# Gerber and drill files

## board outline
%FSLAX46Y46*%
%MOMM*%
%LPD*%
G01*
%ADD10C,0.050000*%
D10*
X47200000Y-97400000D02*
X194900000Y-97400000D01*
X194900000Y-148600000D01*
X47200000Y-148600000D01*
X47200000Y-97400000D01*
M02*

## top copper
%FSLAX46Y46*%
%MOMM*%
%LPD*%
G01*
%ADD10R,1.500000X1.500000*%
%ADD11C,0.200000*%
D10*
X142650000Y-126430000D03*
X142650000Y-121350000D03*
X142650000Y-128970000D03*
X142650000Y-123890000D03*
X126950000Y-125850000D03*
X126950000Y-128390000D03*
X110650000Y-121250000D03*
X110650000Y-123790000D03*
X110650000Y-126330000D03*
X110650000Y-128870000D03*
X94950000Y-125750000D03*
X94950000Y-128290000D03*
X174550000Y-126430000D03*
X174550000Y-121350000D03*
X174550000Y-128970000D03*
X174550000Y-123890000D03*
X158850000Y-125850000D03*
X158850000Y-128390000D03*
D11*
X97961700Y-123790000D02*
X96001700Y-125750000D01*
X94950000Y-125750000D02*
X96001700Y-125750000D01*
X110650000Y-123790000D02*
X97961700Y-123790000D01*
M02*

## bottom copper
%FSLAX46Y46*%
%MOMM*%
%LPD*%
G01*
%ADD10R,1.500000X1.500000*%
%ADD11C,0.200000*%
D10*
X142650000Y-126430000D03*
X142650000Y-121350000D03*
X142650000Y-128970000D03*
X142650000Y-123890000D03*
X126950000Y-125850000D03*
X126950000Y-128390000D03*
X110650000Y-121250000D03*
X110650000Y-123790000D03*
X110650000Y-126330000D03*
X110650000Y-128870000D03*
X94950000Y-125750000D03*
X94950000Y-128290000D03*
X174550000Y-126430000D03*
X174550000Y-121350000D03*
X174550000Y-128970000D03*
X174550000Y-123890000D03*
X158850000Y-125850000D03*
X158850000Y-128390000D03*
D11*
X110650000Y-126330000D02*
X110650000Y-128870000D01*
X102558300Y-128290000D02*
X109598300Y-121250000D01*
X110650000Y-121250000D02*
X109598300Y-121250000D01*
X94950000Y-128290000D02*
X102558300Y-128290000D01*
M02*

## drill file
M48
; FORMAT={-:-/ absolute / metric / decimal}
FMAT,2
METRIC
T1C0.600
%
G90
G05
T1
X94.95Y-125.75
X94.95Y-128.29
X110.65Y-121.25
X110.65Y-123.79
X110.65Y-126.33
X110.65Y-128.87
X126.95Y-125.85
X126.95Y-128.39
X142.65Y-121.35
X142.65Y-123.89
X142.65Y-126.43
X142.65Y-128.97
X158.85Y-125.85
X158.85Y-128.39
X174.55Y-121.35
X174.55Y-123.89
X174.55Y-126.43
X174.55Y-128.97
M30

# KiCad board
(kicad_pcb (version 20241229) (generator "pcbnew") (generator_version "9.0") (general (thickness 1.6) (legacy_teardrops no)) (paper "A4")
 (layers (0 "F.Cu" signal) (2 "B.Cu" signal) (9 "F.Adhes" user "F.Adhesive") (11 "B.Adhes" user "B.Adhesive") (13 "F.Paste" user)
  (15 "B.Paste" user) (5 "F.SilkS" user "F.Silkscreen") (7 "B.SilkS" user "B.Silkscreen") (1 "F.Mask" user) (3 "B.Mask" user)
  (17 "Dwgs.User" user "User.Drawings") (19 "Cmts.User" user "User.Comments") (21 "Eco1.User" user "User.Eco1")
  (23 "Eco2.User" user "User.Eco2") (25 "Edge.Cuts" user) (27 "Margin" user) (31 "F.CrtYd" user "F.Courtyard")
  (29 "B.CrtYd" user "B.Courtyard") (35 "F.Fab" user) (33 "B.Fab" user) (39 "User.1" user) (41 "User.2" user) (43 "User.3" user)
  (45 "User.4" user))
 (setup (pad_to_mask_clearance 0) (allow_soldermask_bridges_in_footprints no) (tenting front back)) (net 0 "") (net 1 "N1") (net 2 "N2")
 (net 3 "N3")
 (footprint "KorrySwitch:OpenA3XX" (layer "F.Cu") (at 124.75 116.85)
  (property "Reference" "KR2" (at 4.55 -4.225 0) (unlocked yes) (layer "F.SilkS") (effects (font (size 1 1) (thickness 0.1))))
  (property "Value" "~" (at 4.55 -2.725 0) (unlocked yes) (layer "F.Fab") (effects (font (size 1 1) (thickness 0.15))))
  (pad "5V_BL" thru_hole rect (at 17.9 9.58) (size 1.5 1.5) (drill 0.6) (layers "*.Cu" "*.Mask") (remove_unused_layers no))
  (pad "5V_TL" thru_hole rect (at 17.9 4.5) (size 1.5 1.5) (drill 0.6) (layers "*.Cu" "*.Mask") (remove_unused_layers no))
  (pad "GND_BL" thru_hole rect (at 17.9 12.12) (size 1.5 1.5) (drill 0.6) (layers "*.Cu" "*.Mask") (remove_unused_layers no))
  (pad "GND_TL" thru_hole rect (at 17.9 7.04) (size 1.5 1.5) (drill 0.6) (layers "*.Cu" "*.Mask") (remove_unused_layers no))
  (pad "SW_IN" thru_hole rect (at 2.2 9) (size 1.5 1.5) (drill 0.6) (layers "*.Cu" "*.Mask") (remove_unused_layers no))
  (pad "SW_OUT" thru_hole rect (at 2.2 11.54) (size 1.5 1.5) (drill 0.6) (layers "*.Cu" "*.Mask") (remove_unused_layers no)))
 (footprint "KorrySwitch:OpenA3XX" (layer "F.Cu") (at 92.75 116.75)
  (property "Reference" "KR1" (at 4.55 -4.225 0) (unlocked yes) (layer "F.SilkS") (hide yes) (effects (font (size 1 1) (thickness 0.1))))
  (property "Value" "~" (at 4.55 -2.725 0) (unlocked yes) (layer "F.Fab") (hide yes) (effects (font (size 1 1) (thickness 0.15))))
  (pad "1" thru_hole rect (at 17.9 4.5) (size 1.5 1.5) (drill 0.6) (layers "*.Cu" "*.Mask") (remove_unused_layers no) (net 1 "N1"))
  (pad "2" thru_hole rect (at 17.9 7.04) (size 1.5 1.5) (drill 0.6) (layers "*.Cu" "*.Mask") (remove_unused_layers no) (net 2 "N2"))
  (pad "3" thru_hole rect (at 17.9 9.58) (size 1.5 1.5) (drill 0.6) (layers "*.Cu" "*.Mask") (remove_unused_layers no) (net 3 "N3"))
  (pad "4" thru_hole rect (at 17.9 12.12) (size 1.5 1.5) (drill 0.6) (layers "*.Cu" "*.Mask") (remove_unused_layers no) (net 3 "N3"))
  (pad "5" thru_hole rect (at 2.2 9) (size 1.5 1.5) (drill 0.6) (layers "*.Cu" "*.Mask") (remove_unused_layers no) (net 2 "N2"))
  (pad "6" thru_hole rect (at 2.2 11.54) (size 1.5 1.5) (drill 0.6) (layers "*.Cu" "*.Mask") (remove_unused_layers no) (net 1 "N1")))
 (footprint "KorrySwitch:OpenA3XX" (layer "F.Cu") (at 156.65 116.85)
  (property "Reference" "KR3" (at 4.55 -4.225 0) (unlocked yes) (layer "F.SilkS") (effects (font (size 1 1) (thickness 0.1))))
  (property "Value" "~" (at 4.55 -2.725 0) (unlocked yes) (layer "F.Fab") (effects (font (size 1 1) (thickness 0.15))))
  (pad "5V_BL" thru_hole rect (at 17.9 9.58) (size 1.5 1.5) (drill 0.6) (layers "*.Cu" "*.Mask") (remove_unused_layers no))
  (pad "5V_TL" thru_hole rect (at 17.9 4.5) (size 1.5 1.5) (drill 0.6) (layers "*.Cu" "*.Mask") (remove_unused_layers no))
  (pad "GND_BL" thru_hole rect (at 17.9 12.12) (size 1.5 1.5) (drill 0.6) (layers "*.Cu" "*.Mask") (remove_unused_layers no))
  (pad "GND_TL" thru_hole rect (at 17.9 7.04) (size 1.5 1.5) (drill 0.6) (layers "*.Cu" "*.Mask") (remove_unused_layers no))
  (pad "SW_IN" thru_hole rect (at 2.2 9) (size 1.5 1.5) (drill 0.6) (layers "*.Cu" "*.Mask") (remove_unused_layers no))
  (pad "SW_OUT" thru_hole rect (at 2.2 11.54) (size 1.5 1.5) (drill 0.6) (layers "*.Cu" "*.Mask") (remove_unused_layers no)))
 (gr_rect (start 47.2 97.4) (end 194.9 148.6) (stroke (width 0.05) (type default)) (fill no) (layer "Edge.Cuts"))
 (segment (start 97.9617 123.79) (end 96.0017 125.75) (width 0.2) (layer "F.Cu") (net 2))
 (segment (start 94.95 125.75) (end 96.0017 125.75) (width 0.2) (layer "F.Cu") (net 2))
 (segment (start 110.65 123.79) (end 97.9617 123.79) (width 0.2) (layer "F.Cu") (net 2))
 (segment (start 110.65 126.33) (end 110.65 128.87) (width 0.2) (layer "B.Cu") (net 3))
 (segment (start 102.5583 128.29) (end 109.5983 121.25) (width 0.2) (layer "B.Cu") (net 1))
 (segment (start 110.65 121.25) (end 109.5983 121.25) (width 0.2) (layer "B.Cu") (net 1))
 (segment (start 94.95 128.29) (end 102.5583 128.29) (width 0.2) (layer "B.Cu") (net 1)))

